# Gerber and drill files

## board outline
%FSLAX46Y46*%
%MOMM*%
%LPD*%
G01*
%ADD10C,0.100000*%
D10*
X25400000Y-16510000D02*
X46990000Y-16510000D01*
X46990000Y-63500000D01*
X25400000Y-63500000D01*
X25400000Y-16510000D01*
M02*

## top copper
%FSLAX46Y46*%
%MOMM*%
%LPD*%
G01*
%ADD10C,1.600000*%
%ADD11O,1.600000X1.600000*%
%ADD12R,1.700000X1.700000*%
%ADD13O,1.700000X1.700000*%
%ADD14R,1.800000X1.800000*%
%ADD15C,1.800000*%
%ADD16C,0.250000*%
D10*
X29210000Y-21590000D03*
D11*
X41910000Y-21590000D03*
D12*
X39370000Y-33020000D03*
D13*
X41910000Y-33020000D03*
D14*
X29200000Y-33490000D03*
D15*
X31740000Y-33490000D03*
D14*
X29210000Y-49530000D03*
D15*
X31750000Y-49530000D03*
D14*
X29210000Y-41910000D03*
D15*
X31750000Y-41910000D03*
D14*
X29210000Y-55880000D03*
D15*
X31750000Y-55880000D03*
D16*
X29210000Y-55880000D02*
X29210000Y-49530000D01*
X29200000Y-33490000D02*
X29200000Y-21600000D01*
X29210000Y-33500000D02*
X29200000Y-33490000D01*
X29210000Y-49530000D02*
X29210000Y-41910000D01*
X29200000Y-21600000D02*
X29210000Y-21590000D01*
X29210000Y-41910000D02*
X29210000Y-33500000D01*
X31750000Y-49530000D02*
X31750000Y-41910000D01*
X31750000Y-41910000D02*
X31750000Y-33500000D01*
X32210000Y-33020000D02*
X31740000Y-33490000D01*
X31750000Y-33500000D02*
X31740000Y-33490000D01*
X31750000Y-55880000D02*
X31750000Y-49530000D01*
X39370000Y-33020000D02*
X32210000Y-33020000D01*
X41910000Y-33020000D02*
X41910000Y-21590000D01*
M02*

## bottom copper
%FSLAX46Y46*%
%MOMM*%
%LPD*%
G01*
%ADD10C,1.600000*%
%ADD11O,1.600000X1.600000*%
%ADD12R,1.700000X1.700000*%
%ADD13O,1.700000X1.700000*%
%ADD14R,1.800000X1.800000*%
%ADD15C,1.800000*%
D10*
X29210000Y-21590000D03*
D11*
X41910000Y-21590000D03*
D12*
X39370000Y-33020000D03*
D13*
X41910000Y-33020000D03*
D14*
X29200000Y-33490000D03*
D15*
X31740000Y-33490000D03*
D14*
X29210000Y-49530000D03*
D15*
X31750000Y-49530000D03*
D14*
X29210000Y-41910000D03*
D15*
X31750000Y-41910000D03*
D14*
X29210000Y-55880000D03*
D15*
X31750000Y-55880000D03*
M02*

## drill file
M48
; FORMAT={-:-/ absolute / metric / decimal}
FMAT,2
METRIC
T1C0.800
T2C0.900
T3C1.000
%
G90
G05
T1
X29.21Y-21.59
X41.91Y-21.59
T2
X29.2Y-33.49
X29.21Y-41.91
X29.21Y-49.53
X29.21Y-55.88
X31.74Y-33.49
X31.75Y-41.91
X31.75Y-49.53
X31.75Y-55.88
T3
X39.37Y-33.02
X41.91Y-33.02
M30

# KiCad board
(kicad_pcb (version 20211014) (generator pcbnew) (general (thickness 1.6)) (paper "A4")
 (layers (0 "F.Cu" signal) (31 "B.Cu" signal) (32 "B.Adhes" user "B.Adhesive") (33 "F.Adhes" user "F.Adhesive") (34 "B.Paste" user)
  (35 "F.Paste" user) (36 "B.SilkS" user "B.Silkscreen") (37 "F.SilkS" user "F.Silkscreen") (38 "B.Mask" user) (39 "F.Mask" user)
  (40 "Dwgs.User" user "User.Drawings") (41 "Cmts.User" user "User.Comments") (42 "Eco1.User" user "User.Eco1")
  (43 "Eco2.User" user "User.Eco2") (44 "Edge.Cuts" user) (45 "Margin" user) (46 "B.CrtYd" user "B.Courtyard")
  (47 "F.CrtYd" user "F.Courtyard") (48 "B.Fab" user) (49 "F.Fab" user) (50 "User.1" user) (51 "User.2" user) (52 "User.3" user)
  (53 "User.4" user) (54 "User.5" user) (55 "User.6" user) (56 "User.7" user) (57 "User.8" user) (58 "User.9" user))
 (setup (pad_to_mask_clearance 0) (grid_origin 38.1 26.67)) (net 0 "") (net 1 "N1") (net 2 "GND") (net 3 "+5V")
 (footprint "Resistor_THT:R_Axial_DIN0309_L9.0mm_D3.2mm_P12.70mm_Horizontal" (layer "F.Cu") (at 29.21 21.59)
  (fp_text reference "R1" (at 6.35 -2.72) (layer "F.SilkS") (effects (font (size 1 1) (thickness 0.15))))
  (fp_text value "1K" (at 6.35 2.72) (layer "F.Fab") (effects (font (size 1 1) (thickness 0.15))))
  (pad "1" thru_hole circle (at 0 0) (size 1.6 1.6) (drill 0.8) (layers *.Cu *.Mask) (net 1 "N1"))
  (pad "2" thru_hole oval (at 12.7 0) (size 1.6 1.6) (drill 0.8) (layers *.Cu *.Mask) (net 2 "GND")))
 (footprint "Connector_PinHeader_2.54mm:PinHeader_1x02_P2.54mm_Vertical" (layer "F.Cu") (at 39.37 33.02 90)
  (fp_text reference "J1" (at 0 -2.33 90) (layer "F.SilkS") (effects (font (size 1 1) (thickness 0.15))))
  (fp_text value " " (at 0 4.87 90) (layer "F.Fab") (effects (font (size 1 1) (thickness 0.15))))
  (pad "1" thru_hole rect (at 0 0 90) (size 1.7 1.7) (drill 1) (layers *.Cu *.Mask) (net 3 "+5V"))
  (pad "2" thru_hole oval (at 0 2.54 90) (size 1.7 1.7) (drill 1) (layers *.Cu *.Mask) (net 2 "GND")))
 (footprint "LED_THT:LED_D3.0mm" (layer "F.Cu") (at 29.2 33.49)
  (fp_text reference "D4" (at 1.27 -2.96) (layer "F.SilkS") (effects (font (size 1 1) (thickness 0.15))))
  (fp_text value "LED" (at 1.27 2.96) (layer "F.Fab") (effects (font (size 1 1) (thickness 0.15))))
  (pad "1" thru_hole rect (at 0 0) (size 1.8 1.8) (drill 0.9) (layers *.Cu *.Mask) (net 1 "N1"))
  (pad "2" thru_hole circle (at 2.54 0) (size 1.8 1.8) (drill 0.9) (layers *.Cu *.Mask) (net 3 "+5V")))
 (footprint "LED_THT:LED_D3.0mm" (layer "F.Cu") (at 29.21 49.53)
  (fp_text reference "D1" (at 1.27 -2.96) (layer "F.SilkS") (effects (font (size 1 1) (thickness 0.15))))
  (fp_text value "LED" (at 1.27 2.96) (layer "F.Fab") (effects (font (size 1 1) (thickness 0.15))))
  (pad "1" thru_hole rect (at 0 0) (size 1.8 1.8) (drill 0.9) (layers *.Cu *.Mask) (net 1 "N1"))
  (pad "2" thru_hole circle (at 2.54 0) (size 1.8 1.8) (drill 0.9) (layers *.Cu *.Mask) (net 3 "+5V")))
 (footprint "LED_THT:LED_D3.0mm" (layer "F.Cu") (at 29.21 41.91)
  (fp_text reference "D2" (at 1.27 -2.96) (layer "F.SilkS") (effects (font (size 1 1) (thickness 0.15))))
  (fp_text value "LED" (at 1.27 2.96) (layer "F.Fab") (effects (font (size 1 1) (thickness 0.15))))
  (pad "1" thru_hole rect (at 0 0) (size 1.8 1.8) (drill 0.9) (layers *.Cu *.Mask) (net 1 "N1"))
  (pad "2" thru_hole circle (at 2.54 0) (size 1.8 1.8) (drill 0.9) (layers *.Cu *.Mask) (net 3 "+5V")))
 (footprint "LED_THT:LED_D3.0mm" (layer "F.Cu") (at 29.21 55.88)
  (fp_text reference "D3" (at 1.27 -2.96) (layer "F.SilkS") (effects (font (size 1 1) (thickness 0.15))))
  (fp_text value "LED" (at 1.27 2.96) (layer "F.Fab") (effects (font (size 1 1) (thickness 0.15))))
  (pad "1" thru_hole rect (at 0 0) (size 1.8 1.8) (drill 0.9) (layers *.Cu *.Mask) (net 1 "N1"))
  (pad "2" thru_hole circle (at 2.54 0) (size 1.8 1.8) (drill 0.9) (layers *.Cu *.Mask) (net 3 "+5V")))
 (gr_rect (start 25.4 16.51) (end 46.99 63.5) (layer "Edge.Cuts") (width 0.1) (fill none))
 (segment (start 29.21 55.88) (end 29.21 49.53) (width 0.25) (layer "F.Cu") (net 1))
 (segment (start 29.2 33.49) (end 29.2 21.6) (width 0.25) (layer "F.Cu") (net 1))
 (segment (start 29.21 33.5) (end 29.2 33.49) (width 0.25) (layer "F.Cu") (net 1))
 (segment (start 29.21 49.53) (end 29.21 41.91) (width 0.25) (layer "F.Cu") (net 1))
 (segment (start 29.2 21.6) (end 29.21 21.59) (width 0.25) (layer "F.Cu") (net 1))
 (segment (start 29.21 41.91) (end 29.21 33.5) (width 0.25) (layer "F.Cu") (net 1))
 (segment (start 31.75 49.53) (end 31.75 41.91) (width 0.25) (layer "F.Cu") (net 3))
 (segment (start 31.75 41.91) (end 31.75 33.5) (width 0.25) (layer "F.Cu") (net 3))
 (segment (start 32.21 33.02) (end 31.74 33.49) (width 0.25) (layer "F.Cu") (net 3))
 (segment (start 31.75 33.5) (end 31.74 33.49) (width 0.25) (layer "F.Cu") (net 3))
 (segment (start 31.75 55.88) (end 31.75 49.53) (width 0.25) (layer "F.Cu") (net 3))
 (segment (start 39.37 33.02) (end 32.21 33.02) (width 0.25) (layer "F.Cu") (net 3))
 (segment (start 41.91 33.02) (end 41.91 21.59) (width 0.25) (layer "F.Cu") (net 2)))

